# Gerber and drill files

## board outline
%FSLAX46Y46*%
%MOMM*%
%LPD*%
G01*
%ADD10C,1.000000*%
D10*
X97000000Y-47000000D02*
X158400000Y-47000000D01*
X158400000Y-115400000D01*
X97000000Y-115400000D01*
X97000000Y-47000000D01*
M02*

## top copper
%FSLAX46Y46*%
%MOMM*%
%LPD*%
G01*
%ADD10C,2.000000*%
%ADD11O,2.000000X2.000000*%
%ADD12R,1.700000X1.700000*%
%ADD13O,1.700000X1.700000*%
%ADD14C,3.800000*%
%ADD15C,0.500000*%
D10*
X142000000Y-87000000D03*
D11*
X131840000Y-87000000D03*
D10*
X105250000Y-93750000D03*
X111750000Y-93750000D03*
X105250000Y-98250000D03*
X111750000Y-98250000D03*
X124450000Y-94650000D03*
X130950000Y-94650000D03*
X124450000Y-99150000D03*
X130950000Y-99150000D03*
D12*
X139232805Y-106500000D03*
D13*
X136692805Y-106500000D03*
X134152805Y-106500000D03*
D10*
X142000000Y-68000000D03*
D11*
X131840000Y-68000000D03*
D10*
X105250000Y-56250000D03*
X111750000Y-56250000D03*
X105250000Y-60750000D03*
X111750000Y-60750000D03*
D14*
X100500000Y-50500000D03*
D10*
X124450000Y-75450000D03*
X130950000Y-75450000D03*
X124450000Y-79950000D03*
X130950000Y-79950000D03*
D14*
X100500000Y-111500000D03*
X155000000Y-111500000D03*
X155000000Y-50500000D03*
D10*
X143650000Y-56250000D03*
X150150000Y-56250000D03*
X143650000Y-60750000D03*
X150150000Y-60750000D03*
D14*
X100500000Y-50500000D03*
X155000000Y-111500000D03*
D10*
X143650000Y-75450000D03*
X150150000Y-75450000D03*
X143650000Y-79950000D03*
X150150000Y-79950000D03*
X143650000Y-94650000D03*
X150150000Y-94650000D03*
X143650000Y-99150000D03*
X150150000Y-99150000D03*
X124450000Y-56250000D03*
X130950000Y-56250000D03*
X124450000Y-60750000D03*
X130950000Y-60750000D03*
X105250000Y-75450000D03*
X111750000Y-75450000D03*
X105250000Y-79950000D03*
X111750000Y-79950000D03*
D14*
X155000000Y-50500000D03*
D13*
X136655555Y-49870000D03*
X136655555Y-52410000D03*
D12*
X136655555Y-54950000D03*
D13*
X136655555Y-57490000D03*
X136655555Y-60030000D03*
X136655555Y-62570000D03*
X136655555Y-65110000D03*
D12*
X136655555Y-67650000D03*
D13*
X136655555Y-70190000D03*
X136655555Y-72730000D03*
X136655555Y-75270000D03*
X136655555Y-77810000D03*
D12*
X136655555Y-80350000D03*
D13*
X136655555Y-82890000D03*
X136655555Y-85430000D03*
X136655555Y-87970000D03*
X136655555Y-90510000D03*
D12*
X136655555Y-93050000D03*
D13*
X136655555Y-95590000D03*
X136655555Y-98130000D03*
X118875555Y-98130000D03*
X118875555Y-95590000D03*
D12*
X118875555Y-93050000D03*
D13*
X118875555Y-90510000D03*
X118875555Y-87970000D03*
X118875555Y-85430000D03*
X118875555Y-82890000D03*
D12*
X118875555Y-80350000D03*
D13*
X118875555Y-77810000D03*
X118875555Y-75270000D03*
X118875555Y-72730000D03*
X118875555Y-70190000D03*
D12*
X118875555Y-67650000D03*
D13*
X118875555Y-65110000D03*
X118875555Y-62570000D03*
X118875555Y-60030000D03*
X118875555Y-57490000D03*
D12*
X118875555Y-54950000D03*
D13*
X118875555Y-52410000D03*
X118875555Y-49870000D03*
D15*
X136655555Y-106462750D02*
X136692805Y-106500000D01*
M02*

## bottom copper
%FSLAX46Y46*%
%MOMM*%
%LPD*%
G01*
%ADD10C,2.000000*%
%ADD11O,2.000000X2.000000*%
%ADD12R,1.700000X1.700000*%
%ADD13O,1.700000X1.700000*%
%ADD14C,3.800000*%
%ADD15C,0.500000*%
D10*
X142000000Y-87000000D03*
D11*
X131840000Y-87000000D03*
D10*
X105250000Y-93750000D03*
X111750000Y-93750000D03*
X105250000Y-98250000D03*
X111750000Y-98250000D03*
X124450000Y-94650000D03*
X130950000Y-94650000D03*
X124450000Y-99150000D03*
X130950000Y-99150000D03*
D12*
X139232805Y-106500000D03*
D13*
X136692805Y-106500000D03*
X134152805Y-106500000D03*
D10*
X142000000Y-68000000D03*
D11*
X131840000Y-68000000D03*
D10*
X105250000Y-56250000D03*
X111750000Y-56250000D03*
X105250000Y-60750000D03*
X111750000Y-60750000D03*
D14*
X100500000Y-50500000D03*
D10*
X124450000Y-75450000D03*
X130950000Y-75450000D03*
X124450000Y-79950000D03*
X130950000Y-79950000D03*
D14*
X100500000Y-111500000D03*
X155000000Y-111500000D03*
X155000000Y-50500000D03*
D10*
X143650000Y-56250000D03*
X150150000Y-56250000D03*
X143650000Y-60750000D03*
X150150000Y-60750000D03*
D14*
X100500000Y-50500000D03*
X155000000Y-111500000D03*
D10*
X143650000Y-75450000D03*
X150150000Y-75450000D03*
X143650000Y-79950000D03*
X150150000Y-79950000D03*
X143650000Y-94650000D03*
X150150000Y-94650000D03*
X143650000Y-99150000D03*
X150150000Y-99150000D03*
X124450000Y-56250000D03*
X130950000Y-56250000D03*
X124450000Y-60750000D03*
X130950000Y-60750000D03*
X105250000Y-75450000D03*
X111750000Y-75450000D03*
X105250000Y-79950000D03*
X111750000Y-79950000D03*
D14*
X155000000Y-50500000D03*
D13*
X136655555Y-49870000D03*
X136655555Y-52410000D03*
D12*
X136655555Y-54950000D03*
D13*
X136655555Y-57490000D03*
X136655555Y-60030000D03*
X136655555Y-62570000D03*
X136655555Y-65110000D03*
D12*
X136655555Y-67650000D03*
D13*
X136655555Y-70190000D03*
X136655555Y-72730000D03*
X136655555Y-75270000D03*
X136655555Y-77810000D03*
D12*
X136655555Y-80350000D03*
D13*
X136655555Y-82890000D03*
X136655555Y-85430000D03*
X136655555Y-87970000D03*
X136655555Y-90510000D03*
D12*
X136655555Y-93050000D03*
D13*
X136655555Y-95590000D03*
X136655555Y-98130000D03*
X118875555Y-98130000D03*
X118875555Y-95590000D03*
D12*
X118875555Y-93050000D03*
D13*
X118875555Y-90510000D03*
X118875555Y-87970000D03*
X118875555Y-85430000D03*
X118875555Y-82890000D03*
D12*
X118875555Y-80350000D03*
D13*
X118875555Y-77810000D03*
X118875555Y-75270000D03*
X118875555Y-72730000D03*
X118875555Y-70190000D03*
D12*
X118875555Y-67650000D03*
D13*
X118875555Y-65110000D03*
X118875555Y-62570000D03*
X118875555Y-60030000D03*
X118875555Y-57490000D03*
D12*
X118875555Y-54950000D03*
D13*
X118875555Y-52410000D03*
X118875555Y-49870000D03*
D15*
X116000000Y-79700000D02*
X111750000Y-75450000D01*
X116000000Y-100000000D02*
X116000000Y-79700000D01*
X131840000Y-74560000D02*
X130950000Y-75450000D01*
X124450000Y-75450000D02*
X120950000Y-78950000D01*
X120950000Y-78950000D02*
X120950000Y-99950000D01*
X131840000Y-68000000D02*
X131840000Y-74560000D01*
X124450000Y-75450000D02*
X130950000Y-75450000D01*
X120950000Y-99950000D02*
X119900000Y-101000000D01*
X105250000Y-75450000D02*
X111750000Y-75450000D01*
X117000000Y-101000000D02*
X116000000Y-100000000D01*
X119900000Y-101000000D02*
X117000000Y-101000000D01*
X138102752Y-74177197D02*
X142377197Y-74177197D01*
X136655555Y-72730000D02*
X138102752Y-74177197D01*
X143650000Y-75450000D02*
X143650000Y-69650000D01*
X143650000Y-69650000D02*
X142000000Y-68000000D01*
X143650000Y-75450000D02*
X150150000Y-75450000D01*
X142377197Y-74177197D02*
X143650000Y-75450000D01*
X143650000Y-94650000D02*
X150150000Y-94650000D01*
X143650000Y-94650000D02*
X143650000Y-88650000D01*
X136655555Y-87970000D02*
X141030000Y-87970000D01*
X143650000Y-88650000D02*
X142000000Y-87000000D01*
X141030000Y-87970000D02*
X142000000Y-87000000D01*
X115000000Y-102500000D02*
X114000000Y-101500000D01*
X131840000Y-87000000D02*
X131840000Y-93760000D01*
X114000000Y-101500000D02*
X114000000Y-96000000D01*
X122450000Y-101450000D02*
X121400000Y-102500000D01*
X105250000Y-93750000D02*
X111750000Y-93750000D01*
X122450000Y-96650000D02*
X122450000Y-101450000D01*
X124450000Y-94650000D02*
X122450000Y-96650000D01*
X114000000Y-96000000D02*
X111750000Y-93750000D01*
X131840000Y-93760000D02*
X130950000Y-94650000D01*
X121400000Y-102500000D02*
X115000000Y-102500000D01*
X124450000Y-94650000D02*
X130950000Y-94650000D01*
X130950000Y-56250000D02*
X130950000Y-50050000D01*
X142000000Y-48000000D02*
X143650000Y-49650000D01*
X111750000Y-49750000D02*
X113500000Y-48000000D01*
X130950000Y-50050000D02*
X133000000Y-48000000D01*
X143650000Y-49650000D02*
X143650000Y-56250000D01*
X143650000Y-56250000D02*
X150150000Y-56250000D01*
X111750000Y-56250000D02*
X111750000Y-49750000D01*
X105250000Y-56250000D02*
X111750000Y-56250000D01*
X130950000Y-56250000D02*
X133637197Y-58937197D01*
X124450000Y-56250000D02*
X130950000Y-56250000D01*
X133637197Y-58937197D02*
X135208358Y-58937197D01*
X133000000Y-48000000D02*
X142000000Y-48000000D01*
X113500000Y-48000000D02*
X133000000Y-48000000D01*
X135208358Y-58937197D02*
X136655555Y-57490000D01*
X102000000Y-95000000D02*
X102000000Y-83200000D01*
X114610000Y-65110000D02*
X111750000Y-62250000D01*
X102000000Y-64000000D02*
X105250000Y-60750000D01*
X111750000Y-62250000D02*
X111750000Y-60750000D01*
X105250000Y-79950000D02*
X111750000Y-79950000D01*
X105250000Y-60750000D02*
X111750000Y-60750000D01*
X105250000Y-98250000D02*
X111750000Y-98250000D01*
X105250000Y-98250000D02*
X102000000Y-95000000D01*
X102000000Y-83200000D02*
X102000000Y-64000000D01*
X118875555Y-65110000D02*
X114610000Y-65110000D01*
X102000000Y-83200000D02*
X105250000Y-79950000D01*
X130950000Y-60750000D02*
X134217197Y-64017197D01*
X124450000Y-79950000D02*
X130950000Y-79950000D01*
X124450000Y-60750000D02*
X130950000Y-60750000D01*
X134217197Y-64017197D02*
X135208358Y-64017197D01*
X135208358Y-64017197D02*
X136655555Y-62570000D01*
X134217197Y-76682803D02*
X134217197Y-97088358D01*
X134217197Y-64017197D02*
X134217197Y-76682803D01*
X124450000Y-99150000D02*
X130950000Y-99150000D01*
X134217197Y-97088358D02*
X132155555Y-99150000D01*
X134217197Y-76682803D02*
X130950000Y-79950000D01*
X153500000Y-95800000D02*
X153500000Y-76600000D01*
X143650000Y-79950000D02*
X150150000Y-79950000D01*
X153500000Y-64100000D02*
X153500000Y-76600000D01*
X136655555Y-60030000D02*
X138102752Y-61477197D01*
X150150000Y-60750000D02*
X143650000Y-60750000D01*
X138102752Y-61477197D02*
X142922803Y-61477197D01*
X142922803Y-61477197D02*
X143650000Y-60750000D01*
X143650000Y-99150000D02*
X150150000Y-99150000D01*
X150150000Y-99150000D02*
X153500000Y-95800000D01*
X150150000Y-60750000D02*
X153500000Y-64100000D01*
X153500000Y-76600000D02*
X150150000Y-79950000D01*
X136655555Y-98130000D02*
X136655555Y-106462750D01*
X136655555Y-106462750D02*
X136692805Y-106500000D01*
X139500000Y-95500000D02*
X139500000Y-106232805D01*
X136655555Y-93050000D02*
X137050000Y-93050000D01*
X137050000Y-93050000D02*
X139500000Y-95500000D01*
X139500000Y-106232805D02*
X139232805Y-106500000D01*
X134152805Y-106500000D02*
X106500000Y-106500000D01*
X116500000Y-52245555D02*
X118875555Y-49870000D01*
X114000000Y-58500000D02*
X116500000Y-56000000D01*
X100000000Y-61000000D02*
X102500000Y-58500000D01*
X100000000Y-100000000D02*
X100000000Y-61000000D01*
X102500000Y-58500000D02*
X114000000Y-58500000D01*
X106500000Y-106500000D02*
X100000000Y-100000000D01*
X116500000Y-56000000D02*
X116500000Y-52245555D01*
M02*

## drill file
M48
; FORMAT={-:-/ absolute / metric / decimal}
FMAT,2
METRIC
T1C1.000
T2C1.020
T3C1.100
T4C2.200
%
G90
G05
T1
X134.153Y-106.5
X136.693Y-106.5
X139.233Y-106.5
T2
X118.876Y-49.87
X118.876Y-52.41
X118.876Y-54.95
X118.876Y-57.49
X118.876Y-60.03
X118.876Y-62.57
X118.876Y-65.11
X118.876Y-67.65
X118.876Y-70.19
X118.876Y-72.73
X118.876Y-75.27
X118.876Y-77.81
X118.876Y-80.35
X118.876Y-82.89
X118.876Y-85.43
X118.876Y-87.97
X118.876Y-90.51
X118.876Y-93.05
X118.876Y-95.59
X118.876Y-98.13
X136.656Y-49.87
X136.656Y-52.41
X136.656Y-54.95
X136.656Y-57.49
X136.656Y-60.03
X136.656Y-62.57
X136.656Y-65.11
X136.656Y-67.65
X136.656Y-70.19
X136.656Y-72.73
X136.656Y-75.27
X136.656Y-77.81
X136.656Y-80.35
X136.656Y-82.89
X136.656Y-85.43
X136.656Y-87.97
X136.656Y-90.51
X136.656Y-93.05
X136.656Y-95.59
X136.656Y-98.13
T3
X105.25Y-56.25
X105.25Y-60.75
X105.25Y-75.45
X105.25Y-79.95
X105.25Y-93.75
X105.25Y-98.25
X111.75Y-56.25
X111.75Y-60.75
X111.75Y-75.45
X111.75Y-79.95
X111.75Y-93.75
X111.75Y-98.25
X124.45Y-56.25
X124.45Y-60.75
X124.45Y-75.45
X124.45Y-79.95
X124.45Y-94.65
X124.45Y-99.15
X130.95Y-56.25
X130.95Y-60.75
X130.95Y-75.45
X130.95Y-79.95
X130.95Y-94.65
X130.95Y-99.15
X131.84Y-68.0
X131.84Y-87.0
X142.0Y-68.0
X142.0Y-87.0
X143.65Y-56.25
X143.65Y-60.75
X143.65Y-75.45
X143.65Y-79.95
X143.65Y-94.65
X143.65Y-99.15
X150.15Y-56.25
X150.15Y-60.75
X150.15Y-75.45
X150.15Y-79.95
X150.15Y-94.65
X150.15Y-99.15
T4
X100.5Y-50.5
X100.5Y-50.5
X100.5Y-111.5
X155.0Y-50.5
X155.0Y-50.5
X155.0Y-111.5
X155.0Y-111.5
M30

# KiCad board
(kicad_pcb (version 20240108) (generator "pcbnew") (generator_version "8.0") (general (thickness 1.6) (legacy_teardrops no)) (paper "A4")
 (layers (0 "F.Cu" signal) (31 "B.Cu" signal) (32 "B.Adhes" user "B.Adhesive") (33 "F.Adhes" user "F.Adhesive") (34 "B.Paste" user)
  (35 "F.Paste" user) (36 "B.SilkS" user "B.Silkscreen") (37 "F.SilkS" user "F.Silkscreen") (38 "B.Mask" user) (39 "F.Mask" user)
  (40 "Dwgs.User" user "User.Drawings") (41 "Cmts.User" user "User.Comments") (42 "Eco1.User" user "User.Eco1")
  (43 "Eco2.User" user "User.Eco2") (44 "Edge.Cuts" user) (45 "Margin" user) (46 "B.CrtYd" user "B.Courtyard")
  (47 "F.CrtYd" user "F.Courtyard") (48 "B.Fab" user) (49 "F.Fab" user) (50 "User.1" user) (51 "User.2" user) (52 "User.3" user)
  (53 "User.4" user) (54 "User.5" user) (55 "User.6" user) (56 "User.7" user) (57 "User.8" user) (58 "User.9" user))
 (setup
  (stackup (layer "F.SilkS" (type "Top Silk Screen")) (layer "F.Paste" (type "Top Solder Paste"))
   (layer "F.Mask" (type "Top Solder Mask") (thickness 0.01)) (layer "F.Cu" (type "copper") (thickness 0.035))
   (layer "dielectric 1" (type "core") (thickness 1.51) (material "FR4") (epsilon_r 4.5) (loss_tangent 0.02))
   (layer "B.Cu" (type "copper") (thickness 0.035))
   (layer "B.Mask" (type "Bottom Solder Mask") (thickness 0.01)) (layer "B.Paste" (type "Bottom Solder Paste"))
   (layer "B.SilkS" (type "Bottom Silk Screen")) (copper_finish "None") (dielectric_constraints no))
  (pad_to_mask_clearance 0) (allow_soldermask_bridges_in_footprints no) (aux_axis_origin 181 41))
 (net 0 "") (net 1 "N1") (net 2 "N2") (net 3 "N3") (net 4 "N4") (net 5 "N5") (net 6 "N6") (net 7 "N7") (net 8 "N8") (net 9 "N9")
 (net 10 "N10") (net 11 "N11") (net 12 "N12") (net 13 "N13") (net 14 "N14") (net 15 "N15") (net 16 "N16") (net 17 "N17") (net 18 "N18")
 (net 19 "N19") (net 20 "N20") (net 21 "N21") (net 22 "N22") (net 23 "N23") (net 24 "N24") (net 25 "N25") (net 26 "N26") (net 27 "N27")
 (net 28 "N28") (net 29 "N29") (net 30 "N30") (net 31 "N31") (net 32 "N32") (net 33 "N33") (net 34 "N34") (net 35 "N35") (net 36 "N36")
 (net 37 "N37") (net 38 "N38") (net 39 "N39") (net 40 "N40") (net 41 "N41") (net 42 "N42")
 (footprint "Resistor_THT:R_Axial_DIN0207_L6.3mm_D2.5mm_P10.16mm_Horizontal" (layer "F.Cu") (at 142 87 180)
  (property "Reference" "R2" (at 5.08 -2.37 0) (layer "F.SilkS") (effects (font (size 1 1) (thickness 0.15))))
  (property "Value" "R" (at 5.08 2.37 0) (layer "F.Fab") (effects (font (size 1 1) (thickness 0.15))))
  (pad "1" thru_hole circle (at 0 0 180) (size 2 1.6) (drill 1.1) (layers "*.Cu" "*.Mask") (remove_unused_layers no) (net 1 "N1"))
  (pad "2" thru_hole oval (at 10.16 0 180) (size 2 2) (drill 1.1) (layers "*.Cu" "*.Mask") (remove_unused_layers no) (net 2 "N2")))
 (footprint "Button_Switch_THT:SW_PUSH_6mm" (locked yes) (layer "F.Cu") (at 105.25 93.75)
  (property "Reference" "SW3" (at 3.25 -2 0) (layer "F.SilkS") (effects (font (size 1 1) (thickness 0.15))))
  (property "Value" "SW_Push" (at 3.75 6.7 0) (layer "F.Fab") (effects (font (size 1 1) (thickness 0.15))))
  (pad "1" thru_hole circle (at 0 0 90) (size 2 2) (drill 1.1) (layers "*.Cu" "*.Mask") (remove_unused_layers no) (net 2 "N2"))
  (pad "1" thru_hole circle (at 6.5 0 90) (size 2 2) (drill 1.1) (layers "*.Cu" "*.Mask") (remove_unused_layers no) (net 2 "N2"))
  (pad "2" thru_hole circle (at 0 4.5 90) (size 2 2) (drill 1.1) (layers "*.Cu" "*.Mask") (remove_unused_layers no) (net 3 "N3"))
  (pad "2" thru_hole circle (at 6.5 4.5 90) (size 2 2) (drill 1.1) (layers "*.Cu" "*.Mask") (remove_unused_layers no) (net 3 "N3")))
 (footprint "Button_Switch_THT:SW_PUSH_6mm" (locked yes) (layer "F.Cu") (at 124.45 94.65)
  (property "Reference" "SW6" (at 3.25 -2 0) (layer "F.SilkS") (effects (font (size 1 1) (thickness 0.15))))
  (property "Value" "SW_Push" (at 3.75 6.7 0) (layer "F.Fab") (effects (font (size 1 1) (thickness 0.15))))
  (pad "1" thru_hole circle (at 0 0 90) (size 2 2) (drill 1.1) (layers "*.Cu" "*.Mask") (remove_unused_layers no) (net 2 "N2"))
  (pad "1" thru_hole circle (at 6.5 0 90) (size 2 2) (drill 1.1) (layers "*.Cu" "*.Mask") (remove_unused_layers no) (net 2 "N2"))
  (pad "2" thru_hole circle (at 0 4.5 90) (size 2 2) (drill 1.1) (layers "*.Cu" "*.Mask") (remove_unused_layers no) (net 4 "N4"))
  (pad "2" thru_hole circle (at 6.5 4.5 90) (size 2 2) (drill 1.1) (layers "*.Cu" "*.Mask") (remove_unused_layers no) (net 4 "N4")))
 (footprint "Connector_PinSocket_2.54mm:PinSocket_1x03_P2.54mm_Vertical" (layer "F.Cu") (at 139.232805 106.5 -90)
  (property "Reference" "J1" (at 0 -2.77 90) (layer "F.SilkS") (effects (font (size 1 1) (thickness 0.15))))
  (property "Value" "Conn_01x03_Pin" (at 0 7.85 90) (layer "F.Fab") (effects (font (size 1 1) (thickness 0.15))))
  (pad "1" thru_hole rect (at 0 0 270) (size 1.7 1.7) (drill 1) (layers "*.Cu" "*.Mask") (remove_unused_layers no) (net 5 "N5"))
  (pad "2" thru_hole oval (at 0 2.54 270) (size 1.7 1.7) (drill 1) (layers "*.Cu" "*.Mask") (remove_unused_layers no) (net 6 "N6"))
  (pad "3" thru_hole oval (at 0 5.08 270) (size 1.7 1.7) (drill 1) (layers "*.Cu" "*.Mask") (remove_unused_layers no) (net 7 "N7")))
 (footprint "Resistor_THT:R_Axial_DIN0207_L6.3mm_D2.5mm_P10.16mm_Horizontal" (layer "F.Cu") (at 142 68 180)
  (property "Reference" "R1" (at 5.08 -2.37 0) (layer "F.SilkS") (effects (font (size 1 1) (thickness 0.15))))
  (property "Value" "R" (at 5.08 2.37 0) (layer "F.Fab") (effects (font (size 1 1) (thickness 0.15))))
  (pad "1" thru_hole circle (at 0 0 180) (size 2 1.6) (drill 1.1) (layers "*.Cu" "*.Mask") (remove_unused_layers no) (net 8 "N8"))
  (pad "2" thru_hole oval (at 10.16 0 180) (size 2 2) (drill 1.1) (layers "*.Cu" "*.Mask") (remove_unused_layers no) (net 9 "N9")))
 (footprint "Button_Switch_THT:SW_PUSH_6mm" (layer "F.Cu") (at 105.25 56.25)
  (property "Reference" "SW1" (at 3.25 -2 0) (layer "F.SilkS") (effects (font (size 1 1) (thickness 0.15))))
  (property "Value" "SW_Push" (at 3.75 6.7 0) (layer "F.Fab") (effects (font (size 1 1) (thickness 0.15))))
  (pad "1" thru_hole circle (at 0 0 90) (size 2 2) (drill 1.1) (layers "*.Cu" "*.Mask") (remove_unused_layers no) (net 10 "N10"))
  (pad "1" thru_hole circle (at 6.5 0 90) (size 2 2) (drill 1.1) (layers "*.Cu" "*.Mask") (remove_unused_layers no) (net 10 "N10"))
  (pad "2" thru_hole circle (at 0 4.5 90) (size 2 2) (drill 1.1) (layers "*.Cu" "*.Mask") (remove_unused_layers no) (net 3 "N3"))
  (pad "2" thru_hole circle (at 6.5 4.5 90) (size 2 2) (drill 1.1) (layers "*.Cu" "*.Mask") (remove_unused_layers no) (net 3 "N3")))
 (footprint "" (layer "F.Cu") (at 100.5 50.5)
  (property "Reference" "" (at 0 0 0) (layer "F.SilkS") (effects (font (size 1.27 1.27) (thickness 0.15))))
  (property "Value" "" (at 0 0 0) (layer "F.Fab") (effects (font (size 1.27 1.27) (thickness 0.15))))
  (pad "1" thru_hole circle (at 0 0) (size 3.8 3.8) (drill 2.2) (layers "*.Cu" "*.Mask") (remove_unused_layers no)))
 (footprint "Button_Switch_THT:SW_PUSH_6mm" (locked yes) (layer "F.Cu") (at 124.45 75.45)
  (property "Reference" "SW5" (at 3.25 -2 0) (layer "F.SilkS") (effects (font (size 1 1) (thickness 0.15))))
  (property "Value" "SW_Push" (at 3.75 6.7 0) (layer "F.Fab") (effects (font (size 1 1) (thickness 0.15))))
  (pad "1" thru_hole circle (at 0 0 90) (size 2 2) (drill 1.1) (layers "*.Cu" "*.Mask") (remove_unused_layers no) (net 9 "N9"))
  (pad "1" thru_hole circle (at 6.5 0 90) (size 2 2) (drill 1.1) (layers "*.Cu" "*.Mask") (remove_unused_layers no) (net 9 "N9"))
  (pad "2" thru_hole circle (at 0 4.5 90) (size 2 2) (drill 1.1) (layers "*.Cu" "*.Mask") (remove_unused_layers no) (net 4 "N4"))
  (pad "2" thru_hole circle (at 6.5 4.5 90) (size 2 2) (drill 1.1) (layers "*.Cu" "*.Mask") (remove_unused_layers no) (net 4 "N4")))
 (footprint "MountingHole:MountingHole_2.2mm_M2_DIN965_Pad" (layer "F.Cu") (at 100.5 111.5)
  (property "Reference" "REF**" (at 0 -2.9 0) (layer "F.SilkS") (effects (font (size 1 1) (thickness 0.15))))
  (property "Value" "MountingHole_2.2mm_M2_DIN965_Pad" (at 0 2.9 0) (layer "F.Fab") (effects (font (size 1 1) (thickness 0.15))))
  (pad "1" thru_hole circle (at 0 0) (size 3.8 3.8) (drill 2.2) (layers "*.Cu" "*.Mask") (remove_unused_layers no)))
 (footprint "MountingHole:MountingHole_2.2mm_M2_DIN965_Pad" (layer "F.Cu") (at 155 111.5)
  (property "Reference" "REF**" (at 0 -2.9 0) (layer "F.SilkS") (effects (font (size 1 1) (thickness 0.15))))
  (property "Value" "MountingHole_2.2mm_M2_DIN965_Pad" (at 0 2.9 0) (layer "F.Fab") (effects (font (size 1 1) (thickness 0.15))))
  (pad "1" thru_hole circle (at 0 0) (size 3.8 3.8) (drill 2.2) (layers "*.Cu" "*.Mask") (remove_unused_layers no)))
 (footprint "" (layer "F.Cu") (at 155 50.5)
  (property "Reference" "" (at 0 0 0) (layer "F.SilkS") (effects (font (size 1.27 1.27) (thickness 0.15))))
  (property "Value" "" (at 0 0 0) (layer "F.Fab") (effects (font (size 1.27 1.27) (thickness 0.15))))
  (pad "1" thru_hole circle (at 0 0) (size 3.8 3.8) (drill 2.2) (layers "*.Cu" "*.Mask") (remove_unused_layers no)))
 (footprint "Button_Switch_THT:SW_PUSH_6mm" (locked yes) (layer "F.Cu") (at 143.65 56.25)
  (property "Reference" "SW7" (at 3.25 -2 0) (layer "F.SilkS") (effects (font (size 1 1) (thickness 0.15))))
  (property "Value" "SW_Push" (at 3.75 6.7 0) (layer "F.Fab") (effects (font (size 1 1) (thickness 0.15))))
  (pad "1" thru_hole circle (at 0 0 90) (size 2 2) (drill 1.1) (layers "*.Cu" "*.Mask") (remove_unused_layers no) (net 10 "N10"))
  (pad "1" thru_hole circle (at 6.5 0 90) (size 2 2) (drill 1.1) (layers "*.Cu" "*.Mask") (remove_unused_layers no) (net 10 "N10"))
  (pad "2" thru_hole circle (at 0 4.5 90) (size 2 2) (drill 1.1) (layers "*.Cu" "*.Mask") (remove_unused_layers no) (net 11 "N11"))
  (pad "2" thru_hole circle (at 6.5 4.5 90) (size 2 2) (drill 1.1) (layers "*.Cu" "*.Mask") (remove_unused_layers no) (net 11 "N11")))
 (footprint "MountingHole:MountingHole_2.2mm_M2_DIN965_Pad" (layer "F.Cu") (at 100.5 50.5)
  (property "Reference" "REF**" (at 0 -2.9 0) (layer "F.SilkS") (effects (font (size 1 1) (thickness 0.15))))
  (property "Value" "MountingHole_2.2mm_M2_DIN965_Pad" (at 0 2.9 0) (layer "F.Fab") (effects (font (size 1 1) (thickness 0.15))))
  (pad "1" thru_hole circle (at 0 0) (size 3.8 3.8) (drill 2.2) (layers "*.Cu" "*.Mask") (remove_unused_layers no)))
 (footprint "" (layer "F.Cu") (at 155 111.5)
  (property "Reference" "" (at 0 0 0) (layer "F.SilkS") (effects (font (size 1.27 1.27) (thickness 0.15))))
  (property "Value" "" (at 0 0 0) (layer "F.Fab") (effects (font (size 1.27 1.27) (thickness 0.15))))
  (pad "1" thru_hole circle (at 0 0) (size 3.8 3.8) (drill 2.2) (layers "*.Cu" "*.Mask") (remove_unused_layers no)))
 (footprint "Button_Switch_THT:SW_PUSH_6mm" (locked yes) (layer "F.Cu") (at 143.65 75.45)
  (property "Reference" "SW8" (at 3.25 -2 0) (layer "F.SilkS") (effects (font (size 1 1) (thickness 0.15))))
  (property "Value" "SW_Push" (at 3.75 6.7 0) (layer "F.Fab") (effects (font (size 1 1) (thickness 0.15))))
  (pad "1" thru_hole circle (at 0 0 90) (size 2 2) (drill 1.1) (layers "*.Cu" "*.Mask") (remove_unused_layers no) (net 8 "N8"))
  (pad "1" thru_hole circle (at 6.5 0 90) (size 2 2) (drill 1.1) (layers "*.Cu" "*.Mask") (remove_unused_layers no) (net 8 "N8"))
  (pad "2" thru_hole circle (at 0 4.5 90) (size 2 2) (drill 1.1) (layers "*.Cu" "*.Mask") (remove_unused_layers no) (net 11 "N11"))
  (pad "2" thru_hole circle (at 6.5 4.5 90) (size 2 2) (drill 1.1) (layers "*.Cu" "*.Mask") (remove_unused_layers no) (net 11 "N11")))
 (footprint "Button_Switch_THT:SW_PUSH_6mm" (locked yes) (layer "F.Cu") (at 143.65 94.65)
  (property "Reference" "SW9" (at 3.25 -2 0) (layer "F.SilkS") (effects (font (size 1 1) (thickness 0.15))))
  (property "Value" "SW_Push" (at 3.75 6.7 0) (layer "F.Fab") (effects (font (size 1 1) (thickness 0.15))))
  (pad "1" thru_hole circle (at 0 0 90) (size 2 2) (drill 1.1) (layers "*.Cu" "*.Mask") (remove_unused_layers no) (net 1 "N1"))
  (pad "1" thru_hole circle (at 6.5 0 90) (size 2 2) (drill 1.1) (layers "*.Cu" "*.Mask") (remove_unused_layers no) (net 1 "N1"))
  (pad "2" thru_hole circle (at 0 4.5 90) (size 2 2) (drill 1.1) (layers "*.Cu" "*.Mask") (remove_unused_layers no) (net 11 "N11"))
  (pad "2" thru_hole circle (at 6.5 4.5 90) (size 2 2) (drill 1.1) (layers "*.Cu" "*.Mask") (remove_unused_layers no) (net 11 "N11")))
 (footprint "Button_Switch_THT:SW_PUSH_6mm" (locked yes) (layer "F.Cu") (at 124.45 56.25)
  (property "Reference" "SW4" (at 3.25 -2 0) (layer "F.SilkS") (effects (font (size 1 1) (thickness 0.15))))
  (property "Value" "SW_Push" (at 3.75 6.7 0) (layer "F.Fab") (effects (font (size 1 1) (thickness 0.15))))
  (pad "1" thru_hole circle (at 0 0 90) (size 2 2) (drill 1.1) (layers "*.Cu" "*.Mask") (remove_unused_layers no) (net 10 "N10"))
  (pad "1" thru_hole circle (at 6.5 0 90) (size 2 2) (drill 1.1) (layers "*.Cu" "*.Mask") (remove_unused_layers no) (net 10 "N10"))
  (pad "2" thru_hole circle (at 0 4.5 90) (size 2 2) (drill 1.1) (layers "*.Cu" "*.Mask") (remove_unused_layers no) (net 4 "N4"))
  (pad "2" thru_hole circle (at 6.5 4.5 90) (size 2 2) (drill 1.1) (layers "*.Cu" "*.Mask") (remove_unused_layers no) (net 4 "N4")))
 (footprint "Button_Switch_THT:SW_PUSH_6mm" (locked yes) (layer "F.Cu") (at 105.25 75.45)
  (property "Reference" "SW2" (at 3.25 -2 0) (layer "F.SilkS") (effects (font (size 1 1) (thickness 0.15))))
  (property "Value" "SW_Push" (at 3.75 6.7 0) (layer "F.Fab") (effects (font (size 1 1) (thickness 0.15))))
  (pad "1" thru_hole circle (at 0 0 90) (size 2 2) (drill 1.1) (layers "*.Cu" "*.Mask") (remove_unused_layers no) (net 9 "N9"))
  (pad "1" thru_hole circle (at 6.5 0 90) (size 2 2) (drill 1.1) (layers "*.Cu" "*.Mask") (remove_unused_layers no) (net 9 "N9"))
  (pad "2" thru_hole circle (at 0 4.5 90) (size 2 2) (drill 1.1) (layers "*.Cu" "*.Mask") (remove_unused_layers no) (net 3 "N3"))
  (pad "2" thru_hole circle (at 6.5 4.5 90) (size 2 2) (drill 1.1) (layers "*.Cu" "*.Mask") (remove_unused_layers no) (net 3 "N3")))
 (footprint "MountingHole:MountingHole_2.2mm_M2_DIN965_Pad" (layer "F.Cu") (at 155 50.5)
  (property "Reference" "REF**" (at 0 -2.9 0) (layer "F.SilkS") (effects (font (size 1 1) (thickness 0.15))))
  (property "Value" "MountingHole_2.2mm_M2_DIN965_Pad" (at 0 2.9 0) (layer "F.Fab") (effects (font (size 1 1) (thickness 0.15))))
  (pad "1" thru_hole circle (at 0 0) (size 3.8 3.8) (drill 2.2) (layers "*.Cu" "*.Mask") (remove_unused_layers no)))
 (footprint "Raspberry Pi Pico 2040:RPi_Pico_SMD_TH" (layer "B.Cu") (at 127.765555 74 180)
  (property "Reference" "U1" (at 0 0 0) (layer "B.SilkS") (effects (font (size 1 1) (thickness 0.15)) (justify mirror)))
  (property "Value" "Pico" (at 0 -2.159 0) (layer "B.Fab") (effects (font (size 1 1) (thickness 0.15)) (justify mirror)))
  (pad "1" thru_hole oval (at -8.89 24.13 180) (size 1.7 1.7) (drill 1.02) (layers "*.Cu" "*.Mask") (remove_unused_layers no) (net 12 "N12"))
  (pad "2" thru_hole oval (at -8.89 21.59 180) (size 1.7 1.7) (drill 1.02) (layers "*.Cu" "*.Mask") (remove_unused_layers no) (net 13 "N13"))
  (pad "3" thru_hole rect (at -8.89 19.05 180) (size 1.7 1.7) (drill 1.02) (layers "*.Cu" "*.Mask") (remove_unused_layers no) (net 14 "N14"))
  (pad "4" thru_hole oval (at -8.89 16.51 180) (size 1.7 1.7) (drill 1.02) (layers "*.Cu" "*.Mask") (remove_unused_layers no) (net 10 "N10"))
  (pad "5" thru_hole oval (at -8.89 13.97 180) (size 1.7 1.7) (drill 1.02) (layers "*.Cu" "*.Mask") (remove_unused_layers no) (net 11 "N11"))
  (pad "6" thru_hole oval (at -8.89 11.43 180) (size 1.7 1.7) (drill 1.02) (layers "*.Cu" "*.Mask") (remove_unused_layers no) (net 4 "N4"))
  (pad "7" thru_hole oval (at -8.89 8.89 180) (size 1.7 1.7) (drill 1.02) (layers "*.Cu" "*.Mask") (remove_unused_layers no) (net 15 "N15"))
  (pad "8" thru_hole rect (at -8.89 6.35 180) (size 1.7 1.7) (drill 1.02) (layers "*.Cu" "*.Mask") (remove_unused_layers no) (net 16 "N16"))
  (pad "9" thru_hole oval (at -8.89 3.81 180) (size 1.7 1.7) (drill 1.02) (layers "*.Cu" "*.Mask") (remove_unused_layers no) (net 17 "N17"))
  (pad "10" thru_hole oval (at -8.89 1.27 180) (size 1.7 1.7) (drill 1.02) (layers "*.Cu" "*.Mask") (remove_unused_layers no) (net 8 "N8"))
  (pad "11" thru_hole oval (at -8.89 -1.27 180) (size 1.7 1.7) (drill 1.02) (layers "*.Cu" "*.Mask") (remove_unused_layers no)
   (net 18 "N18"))
  (pad "12" thru_hole oval (at -8.89 -3.81 180) (size 1.7 1.7) (drill 1.02) (layers "*.Cu" "*.Mask") (remove_unused_layers no)
   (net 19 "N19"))
  (pad "13" thru_hole rect (at -8.89 -6.35 180) (size 1.7 1.7) (drill 1.02) (layers "*.Cu" "*.Mask") (remove_unused_layers no)
   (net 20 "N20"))
  (pad "14" thru_hole oval (at -8.89 -8.89 180) (size 1.7 1.7) (drill 1.02) (layers "*.Cu" "*.Mask") (remove_unused_layers no)
   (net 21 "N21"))
  (pad "15" thru_hole oval (at -8.89 -11.43 180) (size 1.7 1.7) (drill 1.02) (layers "*.Cu" "*.Mask") (remove_unused_layers no)
   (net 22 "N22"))
  (pad "16" thru_hole oval (at -8.89 -13.97 180) (size 1.7 1.7) (drill 1.02) (layers "*.Cu" "*.Mask") (remove_unused_layers no) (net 1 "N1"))
  (pad "17" thru_hole oval (at -8.89 -16.51 180) (size 1.7 1.7) (drill 1.02) (layers "*.Cu" "*.Mask") (remove_unused_layers no)
   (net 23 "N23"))
  (pad "18" thru_hole rect (at -8.89 -19.05 180) (size 1.7 1.7) (drill 1.02) (layers "*.Cu" "*.Mask") (remove_unused_layers no) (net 5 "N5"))
  (pad "19" thru_hole oval (at -8.89 -21.59 180) (size 1.7 1.7) (drill 1.02) (layers "*.Cu" "*.Mask") (remove_unused_layers no)
   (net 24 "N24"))
  (pad "20" thru_hole oval (at -8.89 -24.13 180) (size 1.7 1.7) (drill 1.02) (layers "*.Cu" "*.Mask") (remove_unused_layers no) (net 6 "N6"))
  (pad "21" thru_hole oval (at 8.89 -24.13 180) (size 1.7 1.7) (drill 1.02) (layers "*.Cu" "*.Mask") (remove_unused_layers no)
   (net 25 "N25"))
  (pad "22" thru_hole oval (at 8.89 -21.59 180) (size 1.7 1.7) (drill 1.02) (layers "*.Cu" "*.Mask") (remove_unused_layers no)
   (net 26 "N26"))
  (pad "23" thru_hole rect (at 8.89 -19.05 180) (size 1.7 1.7) (drill 1.02) (layers "*.Cu" "*.Mask") (remove_unused_layers no)
   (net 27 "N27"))
  (pad "24" thru_hole oval (at 8.89 -16.51 180) (size 1.7 1.7) (drill 1.02) (layers "*.Cu" "*.Mask") (remove_unused_layers no)
   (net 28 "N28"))
  (pad "25" thru_hole oval (at 8.89 -13.97 180) (size 1.7 1.7) (drill 1.02) (layers "*.Cu" "*.Mask") (remove_unused_layers no)
   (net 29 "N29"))
  (pad "26" thru_hole oval (at 8.89 -11.43 180) (size 1.7 1.7) (drill 1.02) (layers "*.Cu" "*.Mask") (remove_unused_layers no)
   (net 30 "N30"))
  (pad "27" thru_hole oval (at 8.89 -8.89 180) (size 1.7 1.7) (drill 1.02) (layers "*.Cu" "*.Mask") (remove_unused_layers no) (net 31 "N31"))
  (pad "28" thru_hole rect (at 8.89 -6.35 180) (size 1.7 1.7) (drill 1.02) (layers "*.Cu" "*.Mask") (remove_unused_layers no) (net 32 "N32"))
  (pad "29" thru_hole oval (at 8.89 -3.81 180) (size 1.7 1.7) (drill 1.02) (layers "*.Cu" "*.Mask") (remove_unused_layers no) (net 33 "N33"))
  (pad "30" thru_hole oval (at 8.89 -1.27 180) (size 1.7 1.7) (drill 1.02) (layers "*.Cu" "*.Mask") (remove_unused_layers no) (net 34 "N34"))
  (pad "31" thru_hole oval (at 8.89 1.27 180) (size 1.7 1.7) (drill 1.02) (layers "*.Cu" "*.Mask") (remove_unused_layers no) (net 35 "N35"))
  (pad "32" thru_hole oval (at 8.89 3.81 180) (size 1.7 1.7) (drill 1.02) (layers "*.Cu" "*.Mask") (remove_unused_layers no) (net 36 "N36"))
  (pad "33" thru_hole rect (at 8.89 6.35 180) (size 1.7 1.7) (drill 1.02) (layers "*.Cu" "*.Mask") (remove_unused_layers no) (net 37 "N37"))
  (pad "34" thru_hole oval (at 8.89 8.89 180) (size 1.7 1.7) (drill 1.02) (layers "*.Cu" "*.Mask") (remove_unused_layers no) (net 3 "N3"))
  (pad "35" thru_hole oval (at 8.89 11.43 180) (size 1.7 1.7) (drill 1.02) (layers "*.Cu" "*.Mask") (remove_unused_layers no) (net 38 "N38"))
  (pad "36" thru_hole oval (at 8.89 13.97 180) (size 1.7 1.7) (drill 1.02) (layers "*.Cu" "*.Mask") (remove_unused_layers no) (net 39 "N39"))
  (pad "37" thru_hole oval (at 8.89 16.51 180) (size 1.7 1.7) (drill 1.02) (layers "*.Cu" "*.Mask") (remove_unused_layers no) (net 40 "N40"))
  (pad "38" thru_hole rect (at 8.89 19.05 180) (size 1.7 1.7) (drill 1.02) (layers "*.Cu" "*.Mask") (remove_unused_layers no) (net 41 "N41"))
  (pad "39" thru_hole oval (at 8.89 21.59 180) (size 1.7 1.7) (drill 1.02) (layers "*.Cu" "*.Mask") (remove_unused_layers no) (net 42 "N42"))
  (pad "40" thru_hole oval (at 8.89 24.13 180) (size 1.7 1.7) (drill 1.02) (layers "*.Cu" "*.Mask") (remove_unused_layers no) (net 7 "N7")))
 (gr_rect (start 97 47) (end 158.4 115.4) (locked yes) (stroke (width 1) (type default)) (fill none) (layer "Edge.Cuts"))
 (segment (start 116 79.7) (end 111.75 75.45) (width 0.5) (layer "B.Cu") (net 9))
 (segment (start 116 100) (end 116 79.7) (width 0.5) (layer "B.Cu") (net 9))
 (segment (start 131.84 74.56) (end 130.95 75.45) (width 0.5) (layer "B.Cu") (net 9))
 (segment (start 124.45 75.45) (end 120.95 78.95) (width 0.5) (layer "B.Cu") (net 9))
 (segment (start 120.95 78.95) (end 120.95 99.95) (width 0.5) (layer "B.Cu") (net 9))
 (segment (start 131.84 68) (end 131.84 74.56) (width 0.5) (layer "B.Cu") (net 9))
 (segment (start 124.45 75.45) (end 130.95 75.45) (width 0.5) (layer "B.Cu") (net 9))
 (segment (start 120.95 99.95) (end 119.9 101) (width 0.5) (layer "B.Cu") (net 9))
 (segment (start 105.25 75.45) (end 111.75 75.45) (width 0.5) (layer "B.Cu") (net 9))
 (segment (start 117 101) (end 116 100) (width 0.5) (layer "B.Cu") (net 9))
 (segment (start 119.9 101) (end 117 101) (width 0.5) (layer "B.Cu") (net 9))
 (segment (start 138.102752 74.177197) (end 142.377197 74.177197) (width 0.5) (layer "B.Cu") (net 8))
 (segment (start 136.655555 72.73) (end 138.102752 74.177197) (width 0.5) (layer "B.Cu") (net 8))
 (segment (start 143.65 75.45) (end 143.65 69.65) (width 0.5) (layer "B.Cu") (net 8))
 (segment (start 143.65 69.65) (end 142 68) (width 0.5) (layer "B.Cu") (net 8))
 (segment (start 143.65 75.45) (end 150.15 75.45) (width 0.5) (layer "B.Cu") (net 8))
 (segment (start 142.377197 74.177197) (end 143.65 75.45) (width 0.5) (layer "B.Cu") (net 8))
 (segment (start 143.65 94.65) (end 150.15 94.65) (width 0.5) (layer "B.Cu") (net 1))
 (segment (start 143.65 94.65) (end 143.65 88.65) (width 0.5) (layer "B.Cu") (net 1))
 (segment (start 136.655555 87.97) (end 141.03 87.97) (width 0.5) (layer "B.Cu") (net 1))
 (segment (start 143.65 88.65) (end 142 87) (width 0.5) (layer "B.Cu") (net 1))
 (segment (start 141.03 87.97) (end 142 87) (width 0.5) (layer "B.Cu") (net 1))
 (segment (start 115 102.5) (end 114 101.5) (width 0.5) (layer "B.Cu") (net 2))
 (segment (start 131.84 87) (end 131.84 93.76) (width 0.5) (layer "B.Cu") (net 2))
 (segment (start 114 101.5) (end 114 96) (width 0.5) (layer "B.Cu") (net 2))
 (segment (start 122.45 101.45) (end 121.4 102.5) (width 0.5) (layer "B.Cu") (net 2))
 (segment (start 105.25 93.75) (end 111.75 93.75) (width 0.5) (layer "B.Cu") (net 2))
 (segment (start 122.45 96.65) (end 122.45 101.45) (width 0.5) (layer "B.Cu") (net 2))
 (segment (start 124.45 94.65) (end 122.45 96.65) (width 0.5) (layer "B.Cu") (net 2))
 (segment (start 114 96) (end 111.75 93.75) (width 0.5) (layer "B.Cu") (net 2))
 (segment (start 131.84 93.76) (end 130.95 94.65) (width 0.5) (layer "B.Cu") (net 2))
 (segment (start 121.4 102.5) (end 115 102.5) (width 0.5) (layer "B.Cu") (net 2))
 (segment (start 124.45 94.65) (end 130.95 94.65) (width 0.5) (layer "B.Cu") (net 2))
 (segment (start 130.95 56.25) (end 130.95 50.05) (width 0.5) (layer "B.Cu") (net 10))
 (segment (start 142 48) (end 143.65 49.65) (width 0.5) (layer "B.Cu") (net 10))
 (segment (start 111.75 49.75) (end 113.5 48) (width 0.5) (layer "B.Cu") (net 10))
 (segment (start 130.95 50.05) (end 133 48) (width 0.5) (layer "B.Cu") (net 10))
 (segment (start 143.65 49.65) (end 143.65 56.25) (width 0.5) (layer "B.Cu") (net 10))
 (segment (start 143.65 56.25) (end 150.15 56.25) (width 0.5) (layer "B.Cu") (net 10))
 (segment (start 111.75 56.25) (end 111.75 49.75) (width 0.5) (layer "B.Cu") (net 10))
 (segment (start 105.25 56.25) (end 111.75 56.25) (width 0.5) (layer "B.Cu") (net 10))
 (segment (start 130.95 56.25) (end 133.637197 58.937197) (width 0.5) (layer "B.Cu") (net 10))
 (segment (start 124.45 56.25) (end 130.95 56.25) (width 0.5) (layer "B.Cu") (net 10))
 (segment (start 133.637197 58.937197) (end 135.208358 58.937197) (width 0.5) (layer "B.Cu") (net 10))
 (segment (start 133 48) (end 142 48) (width 0.5) (layer "B.Cu") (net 10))
 (segment (start 113.5 48) (end 133 48) (width 0.5) (layer "B.Cu") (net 10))
 (segment (start 135.208358 58.937197) (end 136.655555 57.49) (width 0.5) (layer "B.Cu") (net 10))
 (segment (start 102 95) (end 102 83.2) (width 0.5) (layer "B.Cu") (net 3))
 (segment (start 114.61 65.11) (end 111.75 62.25) (width 0.5) (layer "B.Cu") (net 3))
 (segment (start 102 64) (end 105.25 60.75) (width 0.5) (layer "B.Cu") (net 3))
 (segment (start 111.75 62.25) (end 111.75 60.75) (width 0.5) (layer "B.Cu") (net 3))
 (segment (start 105.25 79.95) (end 111.75 79.95) (width 0.5) (layer "B.Cu") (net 3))
 (segment (start 105.25 60.75) (end 111.75 60.75) (width 0.5) (layer "B.Cu") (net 3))
 (segment (start 105.25 98.25) (end 111.75 98.25) (width 0.5) (layer "B.Cu") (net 3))
 (segment (start 105.25 98.25) (end 102 95) (width 0.5) (layer "B.Cu") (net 3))
 (segment (start 102 83.2) (end 102 64) (width 0.5) (layer "B.Cu") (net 3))
 (segment (start 118.875555 65.11) (end 114.61 65.11) (width 0.5) (layer "B.Cu") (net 3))
 (segment (start 102 83.2) (end 105.25 79.95) (width 0.5) (layer "B.Cu") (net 3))
 (segment (start 130.95 60.75) (end 134.217197 64.017197) (width 0.5) (layer "B.Cu") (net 4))
 (segment (start 124.45 79.95) (end 130.95 79.95) (width 0.5) (layer "B.Cu") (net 4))
 (segment (start 124.45 60.75) (end 130.95 60.75) (width 0.5) (layer "B.Cu") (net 4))
 (segment (start 134.217197 64.017197) (end 135.208358 64.017197) (width 0.5) (layer "B.Cu") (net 4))
 (segment (start 135.208358 64.017197) (end 136.655555 62.57) (width 0.5) (layer "B.Cu") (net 4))
 (segment (start 134.217197 76.682803) (end 134.217197 97.088358) (width 0.5) (layer "B.Cu") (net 4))
 (segment (start 134.217197 64.017197) (end 134.217197 76.682803) (width 0.5) (layer "B.Cu") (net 4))
 (segment (start 124.45 99.15) (end 130.95 99.15) (width 0.5) (layer "B.Cu") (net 4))
 (segment (start 134.217197 97.088358) (end 132.155555 99.15) (width 0.5) (layer "B.Cu") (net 4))
 (segment (start 134.217197 76.682803) (end 130.95 79.95) (width 0.5) (layer "B.Cu") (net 4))
 (segment (start 153.5 95.8) (end 153.5 76.6) (width 0.5) (layer "B.Cu") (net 11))
 (segment (start 143.65 79.95) (end 150.15 79.95) (width 0.5) (layer "B.Cu") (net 11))
 (segment (start 153.5 64.1) (end 153.5 76.6) (width 0.5) (layer "B.Cu") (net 11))
 (segment (start 136.655555 60.03) (end 138.102752 61.477197) (width 0.5) (layer "B.Cu") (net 11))
 (segment (start 150.15 60.75) (end 143.65 60.75) (width 0.5) (layer "B.Cu") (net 11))
 (segment (start 138.102752 61.477197) (end 142.922803 61.477197) (width 0.5) (layer "B.Cu") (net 11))
 (segment (start 142.922803 61.477197) (end 143.65 60.75) (width 0.5) (layer "B.Cu") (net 11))
 (segment (start 143.65 99.15) (end 150.15 99.15) (width 0.5) (layer "B.Cu") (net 11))
 (segment (start 150.15 99.15) (end 153.5 95.8) (width 0.5) (layer "B.Cu") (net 11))
 (segment (start 150.15 60.75) (end 153.5 64.1) (width 0.5) (layer "B.Cu") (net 11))
 (segment (start 153.5 76.6) (end 150.15 79.95) (width 0.5) (layer "B.Cu") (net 11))
 (segment (start 136.655555 106.46275) (end 136.692805 106.5) (width 0.5) (layer "F.Cu") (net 6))
 (segment (start 136.655555 98.13) (end 136.655555 106.46275) (width 0.5) (layer "B.Cu") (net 6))
 (segment (start 136.655555 106.46275) (end 136.692805 106.5) (width 0.5) (layer "B.Cu") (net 6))
 (segment (start 139.5 95.5) (end 139.5 106.232805) (width 0.5) (layer "B.Cu") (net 5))
 (segment (start 136.655555 93.05) (end 137.05 93.05) (width 0.5) (layer "B.Cu") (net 5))
 (segment (start 137.05 93.05) (end 139.5 95.5) (width 0.5) (layer "B.Cu") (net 5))
 (segment (start 139.5 106.232805) (end 139.232805 106.5) (width 0.5) (layer "B.Cu") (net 5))
 (segment (start 134.152805 106.5) (end 106.5 106.5) (width 0.5) (layer "B.Cu") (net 7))
 (segment (start 116.5 52.245555) (end 118.875555 49.87) (width 0.5) (layer "B.Cu") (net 7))
 (segment (start 114 58.5) (end 116.5 56) (width 0.5) (layer "B.Cu") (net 7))
 (segment (start 100 61) (end 102.5 58.5) (width 0.5) (layer "B.Cu") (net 7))
 (segment (start 100 100) (end 100 61) (width 0.5) (layer "B.Cu") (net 7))
 (segment (start 102.5 58.5) (end 114 58.5) (width 0.5) (layer "B.Cu") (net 7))
 (segment (start 106.5 106.5) (end 100 100) (width 0.5) (layer "B.Cu") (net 7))
 (segment (start 116.5 56) (end 116.5 52.245555) (width 0.5) (layer "B.Cu") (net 7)))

